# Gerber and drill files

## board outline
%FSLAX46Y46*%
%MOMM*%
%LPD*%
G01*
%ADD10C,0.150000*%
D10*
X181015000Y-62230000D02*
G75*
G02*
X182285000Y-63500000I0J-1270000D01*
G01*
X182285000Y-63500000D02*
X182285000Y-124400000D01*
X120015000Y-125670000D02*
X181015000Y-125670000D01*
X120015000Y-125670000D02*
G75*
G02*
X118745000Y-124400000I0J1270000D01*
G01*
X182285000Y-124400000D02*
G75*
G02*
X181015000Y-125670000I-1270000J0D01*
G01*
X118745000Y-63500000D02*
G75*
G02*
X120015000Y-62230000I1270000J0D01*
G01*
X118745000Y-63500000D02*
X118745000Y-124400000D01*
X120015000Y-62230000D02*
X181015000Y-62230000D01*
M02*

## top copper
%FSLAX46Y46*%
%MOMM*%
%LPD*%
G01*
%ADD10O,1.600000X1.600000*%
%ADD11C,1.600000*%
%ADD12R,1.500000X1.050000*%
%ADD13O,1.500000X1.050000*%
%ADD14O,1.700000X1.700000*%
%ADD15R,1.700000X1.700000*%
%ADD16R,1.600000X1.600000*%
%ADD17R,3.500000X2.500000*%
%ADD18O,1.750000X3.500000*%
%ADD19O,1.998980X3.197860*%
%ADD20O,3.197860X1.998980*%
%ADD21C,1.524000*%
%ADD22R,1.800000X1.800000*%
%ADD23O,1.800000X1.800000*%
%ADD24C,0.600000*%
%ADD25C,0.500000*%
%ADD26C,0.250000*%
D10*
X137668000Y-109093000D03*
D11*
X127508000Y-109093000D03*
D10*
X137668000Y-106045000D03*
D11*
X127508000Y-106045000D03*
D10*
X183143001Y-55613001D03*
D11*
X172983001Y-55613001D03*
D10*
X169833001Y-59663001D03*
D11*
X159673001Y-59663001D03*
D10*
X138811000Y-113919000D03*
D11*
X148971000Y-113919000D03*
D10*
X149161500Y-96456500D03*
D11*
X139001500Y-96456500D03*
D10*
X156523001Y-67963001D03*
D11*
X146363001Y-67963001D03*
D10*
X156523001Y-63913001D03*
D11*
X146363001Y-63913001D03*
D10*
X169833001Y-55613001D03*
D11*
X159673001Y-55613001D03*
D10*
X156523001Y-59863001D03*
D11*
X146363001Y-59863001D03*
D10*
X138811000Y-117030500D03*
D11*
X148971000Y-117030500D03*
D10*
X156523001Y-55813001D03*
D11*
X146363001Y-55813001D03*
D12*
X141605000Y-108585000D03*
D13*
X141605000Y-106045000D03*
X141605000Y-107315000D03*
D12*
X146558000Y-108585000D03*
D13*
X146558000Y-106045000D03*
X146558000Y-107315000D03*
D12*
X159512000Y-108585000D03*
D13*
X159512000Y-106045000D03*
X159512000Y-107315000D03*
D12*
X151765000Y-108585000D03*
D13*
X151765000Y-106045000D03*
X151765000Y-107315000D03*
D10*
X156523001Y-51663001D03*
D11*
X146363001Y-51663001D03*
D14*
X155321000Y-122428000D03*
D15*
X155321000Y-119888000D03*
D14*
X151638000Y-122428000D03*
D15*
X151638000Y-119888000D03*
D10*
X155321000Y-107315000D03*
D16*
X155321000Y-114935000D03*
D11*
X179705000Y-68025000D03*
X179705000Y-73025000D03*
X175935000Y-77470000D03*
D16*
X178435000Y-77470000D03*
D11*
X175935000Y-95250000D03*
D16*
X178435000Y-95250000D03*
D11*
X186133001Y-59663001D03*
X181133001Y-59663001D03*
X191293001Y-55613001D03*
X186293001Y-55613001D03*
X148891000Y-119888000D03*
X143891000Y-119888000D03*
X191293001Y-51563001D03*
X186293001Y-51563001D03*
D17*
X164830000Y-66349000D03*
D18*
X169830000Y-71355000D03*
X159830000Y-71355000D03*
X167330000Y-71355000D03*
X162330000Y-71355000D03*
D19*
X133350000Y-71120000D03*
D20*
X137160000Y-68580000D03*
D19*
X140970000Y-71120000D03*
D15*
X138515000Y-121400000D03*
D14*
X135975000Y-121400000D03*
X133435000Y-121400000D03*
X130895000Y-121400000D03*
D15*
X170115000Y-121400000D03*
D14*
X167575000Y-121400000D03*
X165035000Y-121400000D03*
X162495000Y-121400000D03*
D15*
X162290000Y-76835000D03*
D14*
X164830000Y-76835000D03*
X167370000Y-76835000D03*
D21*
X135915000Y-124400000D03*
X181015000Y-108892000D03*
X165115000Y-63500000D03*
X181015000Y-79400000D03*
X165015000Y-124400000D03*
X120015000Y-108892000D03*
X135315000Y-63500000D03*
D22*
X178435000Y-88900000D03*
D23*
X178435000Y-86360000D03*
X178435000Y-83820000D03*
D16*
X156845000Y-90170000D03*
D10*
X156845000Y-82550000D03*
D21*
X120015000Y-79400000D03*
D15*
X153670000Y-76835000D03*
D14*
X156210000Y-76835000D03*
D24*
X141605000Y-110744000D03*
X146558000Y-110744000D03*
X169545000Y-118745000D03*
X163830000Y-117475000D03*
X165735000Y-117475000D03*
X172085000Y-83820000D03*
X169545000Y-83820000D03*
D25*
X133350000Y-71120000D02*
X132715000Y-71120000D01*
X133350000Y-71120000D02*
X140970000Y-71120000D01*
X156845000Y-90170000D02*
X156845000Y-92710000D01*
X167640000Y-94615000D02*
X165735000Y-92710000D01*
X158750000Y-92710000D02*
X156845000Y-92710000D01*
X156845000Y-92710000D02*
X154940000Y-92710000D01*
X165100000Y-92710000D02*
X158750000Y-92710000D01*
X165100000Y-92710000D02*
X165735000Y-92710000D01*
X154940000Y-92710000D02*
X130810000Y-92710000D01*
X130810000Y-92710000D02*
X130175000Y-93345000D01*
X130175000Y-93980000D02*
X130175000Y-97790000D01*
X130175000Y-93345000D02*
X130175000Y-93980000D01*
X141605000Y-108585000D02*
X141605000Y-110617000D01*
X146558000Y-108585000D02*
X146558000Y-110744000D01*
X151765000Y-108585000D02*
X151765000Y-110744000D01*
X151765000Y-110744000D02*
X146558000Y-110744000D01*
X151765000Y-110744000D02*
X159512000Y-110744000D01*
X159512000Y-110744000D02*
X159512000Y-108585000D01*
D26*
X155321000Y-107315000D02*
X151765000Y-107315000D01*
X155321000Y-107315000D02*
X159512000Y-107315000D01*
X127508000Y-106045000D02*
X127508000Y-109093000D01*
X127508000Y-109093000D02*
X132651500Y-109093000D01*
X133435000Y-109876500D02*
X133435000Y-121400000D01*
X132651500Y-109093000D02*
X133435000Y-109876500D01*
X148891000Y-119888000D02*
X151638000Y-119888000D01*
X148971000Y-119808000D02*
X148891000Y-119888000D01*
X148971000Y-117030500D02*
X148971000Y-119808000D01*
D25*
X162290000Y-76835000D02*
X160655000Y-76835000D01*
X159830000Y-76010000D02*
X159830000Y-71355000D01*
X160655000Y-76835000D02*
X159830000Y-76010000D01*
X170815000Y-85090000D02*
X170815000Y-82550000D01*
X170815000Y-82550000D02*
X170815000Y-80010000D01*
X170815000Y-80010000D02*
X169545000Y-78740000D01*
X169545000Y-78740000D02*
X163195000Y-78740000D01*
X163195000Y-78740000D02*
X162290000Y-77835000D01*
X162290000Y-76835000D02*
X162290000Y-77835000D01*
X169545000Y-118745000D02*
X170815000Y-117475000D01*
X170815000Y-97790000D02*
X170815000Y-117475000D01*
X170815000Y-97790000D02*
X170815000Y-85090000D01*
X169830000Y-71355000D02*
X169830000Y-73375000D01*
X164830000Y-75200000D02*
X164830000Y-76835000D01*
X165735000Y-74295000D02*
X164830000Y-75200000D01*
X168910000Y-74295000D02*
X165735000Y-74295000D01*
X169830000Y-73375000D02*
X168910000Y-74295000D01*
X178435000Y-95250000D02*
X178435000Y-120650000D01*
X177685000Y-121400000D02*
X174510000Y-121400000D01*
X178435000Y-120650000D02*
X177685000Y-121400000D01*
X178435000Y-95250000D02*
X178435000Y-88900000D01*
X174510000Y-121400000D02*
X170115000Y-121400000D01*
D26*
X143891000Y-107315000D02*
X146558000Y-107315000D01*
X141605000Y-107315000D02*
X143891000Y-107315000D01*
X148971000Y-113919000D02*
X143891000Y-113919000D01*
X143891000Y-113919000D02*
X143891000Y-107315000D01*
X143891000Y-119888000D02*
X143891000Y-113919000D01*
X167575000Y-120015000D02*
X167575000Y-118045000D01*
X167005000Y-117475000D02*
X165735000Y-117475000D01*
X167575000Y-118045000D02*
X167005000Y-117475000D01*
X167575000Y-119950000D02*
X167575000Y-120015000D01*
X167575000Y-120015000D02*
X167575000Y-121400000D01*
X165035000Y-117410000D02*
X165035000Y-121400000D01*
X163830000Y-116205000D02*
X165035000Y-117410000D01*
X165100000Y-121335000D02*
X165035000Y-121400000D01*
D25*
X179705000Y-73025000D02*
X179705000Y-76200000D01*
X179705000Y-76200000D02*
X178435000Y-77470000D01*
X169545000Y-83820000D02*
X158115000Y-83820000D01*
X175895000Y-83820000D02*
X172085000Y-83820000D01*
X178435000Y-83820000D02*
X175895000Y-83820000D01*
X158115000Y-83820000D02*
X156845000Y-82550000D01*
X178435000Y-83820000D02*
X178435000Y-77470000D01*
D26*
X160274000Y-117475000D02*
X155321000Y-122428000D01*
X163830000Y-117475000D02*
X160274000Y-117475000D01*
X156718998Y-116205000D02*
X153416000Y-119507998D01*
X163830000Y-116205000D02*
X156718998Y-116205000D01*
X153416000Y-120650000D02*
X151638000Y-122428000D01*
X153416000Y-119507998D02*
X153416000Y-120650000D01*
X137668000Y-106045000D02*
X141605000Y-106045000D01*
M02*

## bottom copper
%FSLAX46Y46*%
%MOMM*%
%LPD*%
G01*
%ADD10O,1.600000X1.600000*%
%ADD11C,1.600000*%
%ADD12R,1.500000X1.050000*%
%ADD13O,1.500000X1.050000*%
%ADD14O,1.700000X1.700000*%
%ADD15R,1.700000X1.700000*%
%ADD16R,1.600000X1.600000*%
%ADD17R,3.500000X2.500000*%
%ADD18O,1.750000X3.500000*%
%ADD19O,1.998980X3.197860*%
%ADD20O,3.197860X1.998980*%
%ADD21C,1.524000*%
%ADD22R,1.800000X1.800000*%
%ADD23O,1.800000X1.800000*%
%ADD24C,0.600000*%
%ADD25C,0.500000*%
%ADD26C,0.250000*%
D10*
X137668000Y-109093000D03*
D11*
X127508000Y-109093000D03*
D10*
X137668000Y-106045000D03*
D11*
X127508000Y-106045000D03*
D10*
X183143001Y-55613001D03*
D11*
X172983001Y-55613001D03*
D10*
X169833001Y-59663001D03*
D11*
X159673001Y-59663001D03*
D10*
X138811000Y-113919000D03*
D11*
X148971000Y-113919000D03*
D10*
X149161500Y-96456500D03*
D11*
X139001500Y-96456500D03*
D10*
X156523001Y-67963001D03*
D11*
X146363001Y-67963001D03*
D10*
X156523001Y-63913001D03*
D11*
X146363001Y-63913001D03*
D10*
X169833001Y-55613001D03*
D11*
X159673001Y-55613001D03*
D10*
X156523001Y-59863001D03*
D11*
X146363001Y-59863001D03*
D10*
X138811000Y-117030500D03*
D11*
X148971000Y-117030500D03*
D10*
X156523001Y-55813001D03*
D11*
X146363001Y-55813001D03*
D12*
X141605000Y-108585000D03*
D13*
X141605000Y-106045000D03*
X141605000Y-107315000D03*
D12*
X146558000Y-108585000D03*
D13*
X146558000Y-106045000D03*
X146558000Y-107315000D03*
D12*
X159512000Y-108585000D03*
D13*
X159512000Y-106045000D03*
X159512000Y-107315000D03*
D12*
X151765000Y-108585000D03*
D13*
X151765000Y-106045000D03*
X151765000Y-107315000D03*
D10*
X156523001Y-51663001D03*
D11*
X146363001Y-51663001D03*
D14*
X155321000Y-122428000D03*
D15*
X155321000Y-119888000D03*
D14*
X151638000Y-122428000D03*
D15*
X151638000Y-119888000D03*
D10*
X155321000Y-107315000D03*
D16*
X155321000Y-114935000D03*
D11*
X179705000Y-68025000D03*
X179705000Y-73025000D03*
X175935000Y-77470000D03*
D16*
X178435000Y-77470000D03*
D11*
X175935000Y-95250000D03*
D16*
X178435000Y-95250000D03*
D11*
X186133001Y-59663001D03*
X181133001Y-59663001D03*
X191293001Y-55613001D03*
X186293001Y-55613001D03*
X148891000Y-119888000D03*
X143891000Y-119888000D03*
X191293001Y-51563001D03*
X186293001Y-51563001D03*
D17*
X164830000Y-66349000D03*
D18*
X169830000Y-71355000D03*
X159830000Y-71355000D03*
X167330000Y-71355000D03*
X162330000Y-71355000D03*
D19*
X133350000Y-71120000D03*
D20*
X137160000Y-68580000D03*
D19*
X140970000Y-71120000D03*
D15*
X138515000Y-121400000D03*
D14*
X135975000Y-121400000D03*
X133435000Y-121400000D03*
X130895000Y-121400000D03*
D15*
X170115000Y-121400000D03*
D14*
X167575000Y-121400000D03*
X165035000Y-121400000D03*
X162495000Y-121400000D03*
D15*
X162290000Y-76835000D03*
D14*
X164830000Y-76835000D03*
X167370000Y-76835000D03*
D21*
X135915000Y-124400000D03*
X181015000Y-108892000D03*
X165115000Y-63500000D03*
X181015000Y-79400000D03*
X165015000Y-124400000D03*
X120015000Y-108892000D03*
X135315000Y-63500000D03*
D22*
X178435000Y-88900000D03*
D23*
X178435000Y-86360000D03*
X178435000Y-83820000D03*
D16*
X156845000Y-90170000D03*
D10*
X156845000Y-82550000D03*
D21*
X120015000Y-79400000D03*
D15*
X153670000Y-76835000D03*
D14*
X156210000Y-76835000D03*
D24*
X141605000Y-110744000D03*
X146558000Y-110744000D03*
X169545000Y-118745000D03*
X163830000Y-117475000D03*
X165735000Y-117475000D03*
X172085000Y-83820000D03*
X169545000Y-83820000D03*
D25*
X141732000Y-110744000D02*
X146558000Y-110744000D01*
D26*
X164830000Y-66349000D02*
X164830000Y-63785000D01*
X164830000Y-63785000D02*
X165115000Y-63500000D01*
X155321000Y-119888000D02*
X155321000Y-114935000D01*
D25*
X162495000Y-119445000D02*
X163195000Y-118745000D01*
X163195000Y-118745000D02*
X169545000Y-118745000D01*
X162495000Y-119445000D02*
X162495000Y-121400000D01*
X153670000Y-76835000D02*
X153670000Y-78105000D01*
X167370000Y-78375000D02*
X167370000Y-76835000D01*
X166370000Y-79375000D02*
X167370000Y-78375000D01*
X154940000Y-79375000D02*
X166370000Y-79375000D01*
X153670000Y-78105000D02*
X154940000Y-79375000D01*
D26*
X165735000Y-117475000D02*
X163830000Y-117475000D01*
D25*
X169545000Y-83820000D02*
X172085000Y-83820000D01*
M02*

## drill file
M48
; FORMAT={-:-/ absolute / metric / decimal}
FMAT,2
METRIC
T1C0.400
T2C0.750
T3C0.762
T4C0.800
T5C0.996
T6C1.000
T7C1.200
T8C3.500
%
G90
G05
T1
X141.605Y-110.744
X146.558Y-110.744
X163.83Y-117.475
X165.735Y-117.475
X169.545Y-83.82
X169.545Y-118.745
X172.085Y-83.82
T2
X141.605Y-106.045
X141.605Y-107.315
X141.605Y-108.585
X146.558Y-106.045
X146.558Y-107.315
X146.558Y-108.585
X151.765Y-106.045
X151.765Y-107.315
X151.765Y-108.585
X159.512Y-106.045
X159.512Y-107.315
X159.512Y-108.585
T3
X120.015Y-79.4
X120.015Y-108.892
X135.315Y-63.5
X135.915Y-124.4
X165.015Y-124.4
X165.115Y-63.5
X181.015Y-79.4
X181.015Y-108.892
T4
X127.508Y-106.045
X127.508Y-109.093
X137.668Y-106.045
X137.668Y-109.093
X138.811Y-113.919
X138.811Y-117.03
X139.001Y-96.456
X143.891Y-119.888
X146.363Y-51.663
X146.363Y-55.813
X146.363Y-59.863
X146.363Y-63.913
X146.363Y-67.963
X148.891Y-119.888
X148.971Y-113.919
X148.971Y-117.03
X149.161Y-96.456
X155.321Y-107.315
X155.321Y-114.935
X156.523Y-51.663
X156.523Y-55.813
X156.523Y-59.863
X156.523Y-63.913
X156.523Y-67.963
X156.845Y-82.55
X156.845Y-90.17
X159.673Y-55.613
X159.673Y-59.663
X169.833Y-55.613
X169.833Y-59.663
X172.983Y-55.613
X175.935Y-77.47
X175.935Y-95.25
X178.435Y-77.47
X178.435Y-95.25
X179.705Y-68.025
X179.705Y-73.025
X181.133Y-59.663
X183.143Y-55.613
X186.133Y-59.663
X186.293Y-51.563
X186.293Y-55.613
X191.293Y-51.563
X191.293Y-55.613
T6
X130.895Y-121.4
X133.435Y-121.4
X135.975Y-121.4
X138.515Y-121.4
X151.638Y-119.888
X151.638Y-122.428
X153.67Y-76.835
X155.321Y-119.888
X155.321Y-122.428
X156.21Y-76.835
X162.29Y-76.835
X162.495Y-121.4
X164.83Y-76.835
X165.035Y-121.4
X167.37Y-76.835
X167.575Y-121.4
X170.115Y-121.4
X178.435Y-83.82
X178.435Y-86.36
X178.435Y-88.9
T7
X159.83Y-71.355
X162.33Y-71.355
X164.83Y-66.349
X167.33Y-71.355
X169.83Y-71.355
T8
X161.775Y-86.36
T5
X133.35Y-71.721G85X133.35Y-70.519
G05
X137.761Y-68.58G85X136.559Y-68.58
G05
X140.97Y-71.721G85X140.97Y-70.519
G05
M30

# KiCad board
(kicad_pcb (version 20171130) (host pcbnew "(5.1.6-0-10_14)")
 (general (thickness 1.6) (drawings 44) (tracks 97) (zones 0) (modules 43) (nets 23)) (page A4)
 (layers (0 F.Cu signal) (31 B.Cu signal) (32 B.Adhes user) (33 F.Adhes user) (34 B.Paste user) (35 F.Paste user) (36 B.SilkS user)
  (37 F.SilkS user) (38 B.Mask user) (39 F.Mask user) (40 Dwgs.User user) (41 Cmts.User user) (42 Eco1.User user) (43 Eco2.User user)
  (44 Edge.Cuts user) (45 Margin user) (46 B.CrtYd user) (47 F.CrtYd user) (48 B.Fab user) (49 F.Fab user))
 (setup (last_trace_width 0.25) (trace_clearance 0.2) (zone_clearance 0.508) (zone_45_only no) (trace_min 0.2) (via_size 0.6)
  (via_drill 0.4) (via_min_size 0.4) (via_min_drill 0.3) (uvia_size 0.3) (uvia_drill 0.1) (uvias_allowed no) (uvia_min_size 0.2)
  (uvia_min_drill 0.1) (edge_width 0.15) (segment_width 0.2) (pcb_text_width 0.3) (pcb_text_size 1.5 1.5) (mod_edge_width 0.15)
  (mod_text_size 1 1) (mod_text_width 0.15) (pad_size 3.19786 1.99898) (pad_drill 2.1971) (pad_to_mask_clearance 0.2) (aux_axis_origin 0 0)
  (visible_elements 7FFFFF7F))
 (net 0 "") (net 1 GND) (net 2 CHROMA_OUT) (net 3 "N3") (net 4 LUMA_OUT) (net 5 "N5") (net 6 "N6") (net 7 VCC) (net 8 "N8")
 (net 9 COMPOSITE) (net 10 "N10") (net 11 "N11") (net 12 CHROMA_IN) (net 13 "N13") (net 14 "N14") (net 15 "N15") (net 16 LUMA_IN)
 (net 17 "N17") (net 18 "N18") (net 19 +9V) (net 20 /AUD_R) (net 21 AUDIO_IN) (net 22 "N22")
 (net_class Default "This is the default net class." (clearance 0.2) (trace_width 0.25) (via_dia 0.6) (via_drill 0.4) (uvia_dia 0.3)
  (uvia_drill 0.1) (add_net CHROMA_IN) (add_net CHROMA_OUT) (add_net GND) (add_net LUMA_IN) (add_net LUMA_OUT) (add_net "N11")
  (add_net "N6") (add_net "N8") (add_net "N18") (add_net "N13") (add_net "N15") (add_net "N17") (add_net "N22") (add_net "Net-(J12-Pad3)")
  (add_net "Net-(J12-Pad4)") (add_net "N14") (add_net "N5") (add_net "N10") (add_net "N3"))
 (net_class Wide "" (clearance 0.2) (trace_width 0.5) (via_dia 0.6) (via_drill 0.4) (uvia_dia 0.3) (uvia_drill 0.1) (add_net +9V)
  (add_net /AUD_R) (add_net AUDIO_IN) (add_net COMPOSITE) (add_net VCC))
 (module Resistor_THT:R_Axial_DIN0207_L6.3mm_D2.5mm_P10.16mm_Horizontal (layer F.Cu) (at 127.508 109.093)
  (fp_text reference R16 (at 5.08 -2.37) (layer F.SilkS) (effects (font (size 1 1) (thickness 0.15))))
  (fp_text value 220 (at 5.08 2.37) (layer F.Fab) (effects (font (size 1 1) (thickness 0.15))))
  (pad 2 thru_hole oval (at 10.16 0) (size 1.6 1.6) (drill 0.8) (layers *.Cu *.Mask) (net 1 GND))
  (pad 1 thru_hole circle (at 0 0) (size 1.6 1.6) (drill 0.8) (layers *.Cu *.Mask) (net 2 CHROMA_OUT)))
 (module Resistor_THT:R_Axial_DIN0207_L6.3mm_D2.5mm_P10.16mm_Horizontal (layer F.Cu) (at 127.508 106.045)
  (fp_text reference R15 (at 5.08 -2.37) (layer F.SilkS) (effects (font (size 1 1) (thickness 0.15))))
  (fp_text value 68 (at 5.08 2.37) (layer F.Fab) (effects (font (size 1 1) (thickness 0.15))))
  (pad 2 thru_hole oval (at 10.16 0) (size 1.6 1.6) (drill 0.8) (layers *.Cu *.Mask) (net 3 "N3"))
  (pad 1 thru_hole circle (at 0 0) (size 1.6 1.6) (drill 0.8) (layers *.Cu *.Mask) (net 2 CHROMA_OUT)))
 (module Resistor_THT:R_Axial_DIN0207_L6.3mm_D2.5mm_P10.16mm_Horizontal (layer F.Cu) (at 172.983001 55.613001)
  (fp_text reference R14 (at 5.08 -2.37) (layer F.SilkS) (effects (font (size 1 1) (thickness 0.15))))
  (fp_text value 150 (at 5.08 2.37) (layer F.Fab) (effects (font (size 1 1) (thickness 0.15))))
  (pad 2 thru_hole oval (at 10.16 0) (size 1.6 1.6) (drill 0.8) (layers *.Cu *.Mask) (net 1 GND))
  (pad 1 thru_hole circle (at 0 0) (size 1.6 1.6) (drill 0.8) (layers *.Cu *.Mask) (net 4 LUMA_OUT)))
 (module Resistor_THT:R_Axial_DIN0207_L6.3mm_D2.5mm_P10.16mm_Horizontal (layer F.Cu) (at 159.673001 59.663001)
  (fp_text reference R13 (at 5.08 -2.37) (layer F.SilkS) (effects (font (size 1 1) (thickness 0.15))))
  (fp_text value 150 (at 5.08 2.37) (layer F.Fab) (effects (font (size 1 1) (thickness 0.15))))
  (pad 2 thru_hole oval (at 10.16 0) (size 1.6 1.6) (drill 0.8) (layers *.Cu *.Mask) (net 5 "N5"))
  (pad 1 thru_hole circle (at 0 0) (size 1.6 1.6) (drill 0.8) (layers *.Cu *.Mask) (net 4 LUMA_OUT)))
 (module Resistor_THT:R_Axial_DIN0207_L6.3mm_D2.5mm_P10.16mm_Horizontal (layer F.Cu) (at 148.971 113.919 180)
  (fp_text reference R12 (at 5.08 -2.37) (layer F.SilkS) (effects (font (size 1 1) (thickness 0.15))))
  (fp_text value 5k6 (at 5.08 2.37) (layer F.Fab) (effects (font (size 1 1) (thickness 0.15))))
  (pad 2 thru_hole oval (at 10.16 0 180) (size 1.6 1.6) (drill 0.8) (layers *.Cu *.Mask) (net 1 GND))
  (pad 1 thru_hole circle (at 0 0 180) (size 1.6 1.6) (drill 0.8) (layers *.Cu *.Mask) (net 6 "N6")))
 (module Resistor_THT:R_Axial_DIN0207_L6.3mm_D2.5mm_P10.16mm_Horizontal (layer F.Cu) (at 139.0015 96.4565)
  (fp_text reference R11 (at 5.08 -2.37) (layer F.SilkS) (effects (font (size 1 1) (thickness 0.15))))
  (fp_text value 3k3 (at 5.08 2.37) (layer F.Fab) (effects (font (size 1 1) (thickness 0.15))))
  (pad 2 thru_hole oval (at 10.16 0) (size 1.6 1.6) (drill 0.8) (layers *.Cu *.Mask) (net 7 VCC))
  (pad 1 thru_hole circle (at 0 0) (size 1.6 1.6) (drill 0.8) (layers *.Cu *.Mask) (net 6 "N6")))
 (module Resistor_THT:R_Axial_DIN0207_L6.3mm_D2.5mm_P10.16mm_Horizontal (layer F.Cu) (at 146.363001 67.963001)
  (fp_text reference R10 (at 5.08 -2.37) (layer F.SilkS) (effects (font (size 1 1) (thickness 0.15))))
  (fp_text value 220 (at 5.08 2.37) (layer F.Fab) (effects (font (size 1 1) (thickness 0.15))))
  (pad 2 thru_hole oval (at 10.16 0) (size 1.6 1.6) (drill 0.8) (layers *.Cu *.Mask) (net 1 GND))
  (pad 1 thru_hole circle (at 0 0) (size 1.6 1.6) (drill 0.8) (layers *.Cu *.Mask) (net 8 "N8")))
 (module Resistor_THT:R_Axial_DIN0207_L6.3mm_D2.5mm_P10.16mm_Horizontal (layer F.Cu) (at 146.363001 63.913001)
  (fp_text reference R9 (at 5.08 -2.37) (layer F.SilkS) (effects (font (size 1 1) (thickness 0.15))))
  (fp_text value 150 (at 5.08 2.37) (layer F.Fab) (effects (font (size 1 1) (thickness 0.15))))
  (pad 2 thru_hole oval (at 10.16 0) (size 1.6 1.6) (drill 0.8) (layers *.Cu *.Mask) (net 1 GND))
  (pad 1 thru_hole circle (at 0 0) (size 1.6 1.6) (drill 0.8) (layers *.Cu *.Mask) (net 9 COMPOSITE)))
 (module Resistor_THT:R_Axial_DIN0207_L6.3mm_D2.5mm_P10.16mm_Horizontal (layer F.Cu) (at 159.673001 55.613001)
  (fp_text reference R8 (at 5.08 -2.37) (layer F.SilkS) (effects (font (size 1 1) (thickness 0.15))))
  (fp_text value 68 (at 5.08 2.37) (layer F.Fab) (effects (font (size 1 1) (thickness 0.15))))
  (pad 2 thru_hole oval (at 10.16 0) (size 1.6 1.6) (drill 0.8) (layers *.Cu *.Mask) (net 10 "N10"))
  (pad 1 thru_hole circle (at 0 0) (size 1.6 1.6) (drill 0.8) (layers *.Cu *.Mask) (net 8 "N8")))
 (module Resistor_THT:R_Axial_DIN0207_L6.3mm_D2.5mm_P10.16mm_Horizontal (layer F.Cu) (at 146.363001 59.863001)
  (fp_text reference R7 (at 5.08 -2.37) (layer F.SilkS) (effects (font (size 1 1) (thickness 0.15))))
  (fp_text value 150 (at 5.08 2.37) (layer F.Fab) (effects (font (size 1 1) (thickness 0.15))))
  (pad 2 thru_hole oval (at 10.16 0) (size 1.6 1.6) (drill 0.8) (layers *.Cu *.Mask) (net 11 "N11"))
  (pad 1 thru_hole circle (at 0 0) (size 1.6 1.6) (drill 0.8) (layers *.Cu *.Mask) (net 9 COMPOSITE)))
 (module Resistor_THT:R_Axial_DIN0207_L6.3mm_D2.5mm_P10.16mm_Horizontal (layer F.Cu) (at 148.971 117.0305 180)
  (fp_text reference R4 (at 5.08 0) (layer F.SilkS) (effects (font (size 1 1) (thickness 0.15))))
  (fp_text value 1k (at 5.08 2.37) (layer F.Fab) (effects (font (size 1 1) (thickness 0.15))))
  (pad 2 thru_hole oval (at 10.16 0 180) (size 1.6 1.6) (drill 0.8) (layers *.Cu *.Mask) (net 1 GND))
  (pad 1 thru_hole circle (at 0 0 180) (size 1.6 1.6) (drill 0.8) (layers *.Cu *.Mask) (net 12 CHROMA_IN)))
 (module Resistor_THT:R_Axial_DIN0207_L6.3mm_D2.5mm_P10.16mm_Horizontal (layer F.Cu) (at 146.363001 55.813001)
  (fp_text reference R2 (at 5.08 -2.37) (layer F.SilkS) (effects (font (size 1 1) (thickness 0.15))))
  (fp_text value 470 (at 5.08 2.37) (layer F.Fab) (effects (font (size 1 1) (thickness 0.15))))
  (pad 2 thru_hole oval (at 10.16 0) (size 1.6 1.6) (drill 0.8) (layers *.Cu *.Mask) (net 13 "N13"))
  (pad 1 thru_hole circle (at 0 0) (size 1.6 1.6) (drill 0.8) (layers *.Cu *.Mask) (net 7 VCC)))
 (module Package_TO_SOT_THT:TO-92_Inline (layer F.Cu) (at 141.605 108.585 90)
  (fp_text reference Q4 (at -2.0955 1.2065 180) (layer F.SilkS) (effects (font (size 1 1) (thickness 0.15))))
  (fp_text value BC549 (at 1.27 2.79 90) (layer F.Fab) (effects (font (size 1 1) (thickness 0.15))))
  (pad 1 thru_hole rect (at 0 0 90) (size 1.05 1.5) (drill 0.75) (layers *.Cu *.Mask) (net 7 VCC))
  (pad 3 thru_hole oval (at 2.54 0 90) (size 1.05 1.5) (drill 0.75) (layers *.Cu *.Mask) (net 3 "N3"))
  (pad 2 thru_hole oval (at 1.27 0 90) (size 1.05 1.5) (drill 0.75) (layers *.Cu *.Mask) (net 6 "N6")))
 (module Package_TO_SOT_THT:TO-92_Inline (layer F.Cu) (at 146.558 108.585 90)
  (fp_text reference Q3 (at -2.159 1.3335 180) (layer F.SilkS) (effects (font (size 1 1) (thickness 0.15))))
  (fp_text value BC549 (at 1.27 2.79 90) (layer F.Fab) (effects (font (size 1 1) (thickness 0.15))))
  (pad 1 thru_hole rect (at 0 0 90) (size 1.05 1.5) (drill 0.75) (layers *.Cu *.Mask) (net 7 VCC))
  (pad 3 thru_hole oval (at 2.54 0 90) (size 1.05 1.5) (drill 0.75) (layers *.Cu *.Mask) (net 10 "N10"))
  (pad 2 thru_hole oval (at 1.27 0 90) (size 1.05 1.5) (drill 0.75) (layers *.Cu *.Mask) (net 6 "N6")))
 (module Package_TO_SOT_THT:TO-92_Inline (layer F.Cu) (at 159.512 108.585 90)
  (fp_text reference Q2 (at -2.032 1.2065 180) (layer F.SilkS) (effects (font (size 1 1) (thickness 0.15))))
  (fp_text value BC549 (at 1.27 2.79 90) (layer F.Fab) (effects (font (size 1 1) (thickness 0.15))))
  (pad 1 thru_hole rect (at 0 0 90) (size 1.05 1.5) (drill 0.75) (layers *.Cu *.Mask) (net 7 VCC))
  (pad 3 thru_hole oval (at 2.54 0 90) (size 1.05 1.5) (drill 0.75) (layers *.Cu *.Mask) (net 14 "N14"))
  (pad 2 thru_hole oval (at 1.27 0 90) (size 1.05 1.5) (drill 0.75) (layers *.Cu *.Mask) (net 13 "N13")))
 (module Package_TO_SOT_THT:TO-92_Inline (layer F.Cu) (at 151.765 108.585 90)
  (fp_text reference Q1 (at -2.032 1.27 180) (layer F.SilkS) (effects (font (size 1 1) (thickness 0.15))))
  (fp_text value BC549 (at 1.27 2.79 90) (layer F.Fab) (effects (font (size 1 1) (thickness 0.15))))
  (pad 1 thru_hole rect (at 0 0 90) (size 1.05 1.5) (drill 0.75) (layers *.Cu *.Mask) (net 7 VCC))
  (pad 3 thru_hole oval (at 2.54 0 90) (size 1.05 1.5) (drill 0.75) (layers *.Cu *.Mask) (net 5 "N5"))
  (pad 2 thru_hole oval (at 1.27 0 90) (size 1.05 1.5) (drill 0.75) (layers *.Cu *.Mask) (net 13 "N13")))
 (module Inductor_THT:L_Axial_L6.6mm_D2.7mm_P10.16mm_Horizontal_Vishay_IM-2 (layer F.Cu) (at 146.363001 51.663001)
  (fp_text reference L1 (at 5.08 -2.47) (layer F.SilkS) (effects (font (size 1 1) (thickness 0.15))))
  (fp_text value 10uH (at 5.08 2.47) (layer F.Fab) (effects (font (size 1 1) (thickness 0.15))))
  (pad 2 thru_hole oval (at 10.16 0) (size 1.6 1.6) (drill 0.8) (layers *.Cu *.Mask) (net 14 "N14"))
  (pad 1 thru_hole circle (at 0 0) (size 1.6 1.6) (drill 0.8) (layers *.Cu *.Mask) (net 11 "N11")))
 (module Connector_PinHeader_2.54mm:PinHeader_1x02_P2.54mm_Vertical (layer F.Cu) (at 155.321 119.888)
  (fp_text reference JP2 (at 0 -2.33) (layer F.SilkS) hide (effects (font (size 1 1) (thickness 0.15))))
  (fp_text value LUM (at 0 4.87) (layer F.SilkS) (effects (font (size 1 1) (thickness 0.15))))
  (pad 2 thru_hole oval (at 0 2.54) (size 1.7 1.7) (drill 1) (layers *.Cu *.Mask) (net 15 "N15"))
  (pad 1 thru_hole rect (at 0 0) (size 1.7 1.7) (drill 1) (layers *.Cu *.Mask) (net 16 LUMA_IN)))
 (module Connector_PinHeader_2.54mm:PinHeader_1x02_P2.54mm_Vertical (layer F.Cu) (at 151.638 119.888)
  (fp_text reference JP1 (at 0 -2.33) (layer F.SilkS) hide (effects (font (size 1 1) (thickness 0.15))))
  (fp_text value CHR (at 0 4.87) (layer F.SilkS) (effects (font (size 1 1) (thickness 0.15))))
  (pad 2 thru_hole oval (at 0 2.54) (size 1.7 1.7) (drill 1) (layers *.Cu *.Mask) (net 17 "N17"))
  (pad 1 thru_hole rect (at 0 0) (size 1.7 1.7) (drill 1) (layers *.Cu *.Mask) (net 12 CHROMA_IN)))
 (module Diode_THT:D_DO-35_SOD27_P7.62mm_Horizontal (layer F.Cu) (at 155.321 114.935 90)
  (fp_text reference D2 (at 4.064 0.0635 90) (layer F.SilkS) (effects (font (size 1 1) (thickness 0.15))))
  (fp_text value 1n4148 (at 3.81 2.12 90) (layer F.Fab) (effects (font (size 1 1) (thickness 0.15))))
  (pad 2 thru_hole oval (at 7.62 0 90) (size 1.6 1.6) (drill 0.8) (layers *.Cu *.Mask) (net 13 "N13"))
  (pad 1 thru_hole rect (at 0 0 90) (size 1.6 1.6) (drill 0.8) (layers *.Cu *.Mask) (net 16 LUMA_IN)))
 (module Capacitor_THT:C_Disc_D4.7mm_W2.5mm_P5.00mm (layer F.Cu) (at 179.705 73.025 90)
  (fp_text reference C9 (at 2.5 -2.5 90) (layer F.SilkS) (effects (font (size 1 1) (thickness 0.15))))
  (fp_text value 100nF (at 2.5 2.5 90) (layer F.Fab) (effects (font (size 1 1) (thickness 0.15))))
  (pad 2 thru_hole circle (at 5 0 90) (size 1.6 1.6) (drill 0.8) (layers *.Cu *.Mask) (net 1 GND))
  (pad 1 thru_hole circle (at 0 0 90) (size 1.6 1.6) (drill 0.8) (layers *.Cu *.Mask) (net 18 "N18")))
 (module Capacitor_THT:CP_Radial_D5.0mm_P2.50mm (layer F.Cu) (at 178.435 77.47 180)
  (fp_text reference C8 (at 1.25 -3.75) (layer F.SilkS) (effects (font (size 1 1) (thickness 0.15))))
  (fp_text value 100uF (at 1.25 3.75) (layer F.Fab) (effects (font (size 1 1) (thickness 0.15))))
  (pad 2 thru_hole circle (at 2.5 0 180) (size 1.6 1.6) (drill 0.8) (layers *.Cu *.Mask) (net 1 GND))
  (pad 1 thru_hole rect (at 0 0 180) (size 1.6 1.6) (drill 0.8) (layers *.Cu *.Mask) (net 18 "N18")))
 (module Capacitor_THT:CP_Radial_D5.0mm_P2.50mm (layer F.Cu) (at 178.435 95.25 180)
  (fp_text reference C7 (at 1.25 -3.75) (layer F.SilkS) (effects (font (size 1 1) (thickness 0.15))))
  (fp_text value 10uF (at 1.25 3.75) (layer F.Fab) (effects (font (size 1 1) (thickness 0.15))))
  (pad 2 thru_hole circle (at 2.5 0 180) (size 1.6 1.6) (drill 0.8) (layers *.Cu *.Mask) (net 1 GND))
  (pad 1 thru_hole rect (at 0 0 180) (size 1.6 1.6) (drill 0.8) (layers *.Cu *.Mask) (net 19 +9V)))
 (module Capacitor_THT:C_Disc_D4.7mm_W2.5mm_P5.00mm (layer F.Cu) (at 181.133001 59.663001)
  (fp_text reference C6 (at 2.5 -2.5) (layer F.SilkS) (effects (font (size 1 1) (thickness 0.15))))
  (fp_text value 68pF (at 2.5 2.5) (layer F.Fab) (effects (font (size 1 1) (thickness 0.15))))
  (pad 2 thru_hole circle (at 5 0) (size 1.6 1.6) (drill 0.8) (layers *.Cu *.Mask) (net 9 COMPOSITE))
  (pad 1 thru_hole circle (at 0 0) (size 1.6 1.6) (drill 0.8) (layers *.Cu *.Mask) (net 8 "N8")))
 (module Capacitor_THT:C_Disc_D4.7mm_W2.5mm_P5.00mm (layer F.Cu) (at 186.293001 55.613001)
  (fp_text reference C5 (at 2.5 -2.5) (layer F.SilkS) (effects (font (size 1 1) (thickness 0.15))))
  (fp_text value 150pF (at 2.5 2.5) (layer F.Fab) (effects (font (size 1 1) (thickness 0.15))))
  (pad 2 thru_hole circle (at 5 0) (size 1.6 1.6) (drill 0.8) (layers *.Cu *.Mask) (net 1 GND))
  (pad 1 thru_hole circle (at 0 0) (size 1.6 1.6) (drill 0.8) (layers *.Cu *.Mask) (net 6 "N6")))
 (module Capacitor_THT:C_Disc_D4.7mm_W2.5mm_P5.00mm (layer F.Cu) (at 143.891 119.888)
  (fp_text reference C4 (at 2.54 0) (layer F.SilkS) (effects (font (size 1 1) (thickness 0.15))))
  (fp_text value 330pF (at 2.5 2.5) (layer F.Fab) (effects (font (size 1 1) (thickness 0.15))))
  (pad 2 thru_hole circle (at 5 0) (size 1.6 1.6) (drill 0.8) (layers *.Cu *.Mask) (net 12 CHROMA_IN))
  (pad 1 thru_hole circle (at 0 0) (size 1.6 1.6) (drill 0.8) (layers *.Cu *.Mask) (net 6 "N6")))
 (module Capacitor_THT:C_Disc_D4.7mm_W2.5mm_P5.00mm (layer F.Cu) (at 186.293001 51.563001)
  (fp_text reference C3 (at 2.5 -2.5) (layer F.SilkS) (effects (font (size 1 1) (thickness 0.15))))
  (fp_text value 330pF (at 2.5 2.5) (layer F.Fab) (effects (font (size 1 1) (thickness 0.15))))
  (pad 2 thru_hole circle (at 5 0) (size 1.6 1.6) (drill 0.8) (layers *.Cu *.Mask) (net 1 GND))
  (pad 1 thru_hole circle (at 0 0) (size 1.6 1.6) (drill 0.8) (layers *.Cu *.Mask) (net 11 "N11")))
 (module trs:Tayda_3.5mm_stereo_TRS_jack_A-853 (layer F.Cu) (at 164.83 67.945)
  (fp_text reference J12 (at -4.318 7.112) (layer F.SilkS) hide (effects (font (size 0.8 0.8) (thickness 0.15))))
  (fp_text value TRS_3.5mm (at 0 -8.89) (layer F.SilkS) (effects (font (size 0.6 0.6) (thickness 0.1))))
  (pad 1 thru_hole rect (at 0 -1.596) (size 3.5 2.5) (drill 1.2) (layers *.Cu *.Mask F.SilkS) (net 1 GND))
  (pad 2 thru_hole oval (at 5 3.41) (size 1.75 3.5) (drill 1.2) (layers *.Cu *.Mask F.SilkS) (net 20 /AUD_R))
  (pad 5 thru_hole oval (at -5 3.41) (size 1.75 3.5) (drill 1.2) (layers *.Cu *.Mask F.SilkS) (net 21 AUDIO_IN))
  (pad 3 thru_hole oval (at 2.5 3.41) (size 1.75 3.5) (drill 1.2) (layers *.Cu *.Mask F.SilkS))
  (pad 4 thru_hole oval (at -2.5 3.41) (size 1.75 3.5) (drill 1.2) (layers *.Cu *.Mask F.SilkS)))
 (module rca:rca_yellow (layer F.Cu) (at 137.16 67.31 180)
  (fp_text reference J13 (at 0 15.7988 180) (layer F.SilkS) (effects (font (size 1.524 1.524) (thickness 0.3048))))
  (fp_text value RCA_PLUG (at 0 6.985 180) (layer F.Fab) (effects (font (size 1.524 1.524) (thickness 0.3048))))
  (pad 2 thru_hole oval (at 3.81 -3.81 180) (size 1.99898 3.19786) (drill oval 0.99568 2.1971) (layers *.Cu *.Mask F.SilkS)
   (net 9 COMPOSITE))
  (pad 1 thru_hole oval (at 0 -1.27 180) (size 3.19786 1.99898) (drill oval 2.1971 0.99568) (layers *.Cu *.Mask F.SilkS) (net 1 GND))
  (pad 2 thru_hole oval (at -3.81 -3.81 180) (size 1.99898 3.19786) (drill oval 0.99568 2.1971) (layers *.Cu *.Mask F.SilkS)
   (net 9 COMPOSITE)))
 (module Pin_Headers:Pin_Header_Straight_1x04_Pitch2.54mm (layer F.Cu) (at 138.515 121.4 270)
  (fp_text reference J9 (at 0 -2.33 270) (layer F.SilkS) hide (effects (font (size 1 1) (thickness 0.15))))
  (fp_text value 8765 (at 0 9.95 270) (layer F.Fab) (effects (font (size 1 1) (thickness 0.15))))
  (pad 1 thru_hole rect (at 0 0 270) (size 1.7 1.7) (drill 1) (layers *.Cu *.Mask) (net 9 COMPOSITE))
  (pad 2 thru_hole oval (at 0 2.54 270) (size 1.7 1.7) (drill 1) (layers *.Cu *.Mask) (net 4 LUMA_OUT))
  (pad 3 thru_hole oval (at 0 5.08 270) (size 1.7 1.7) (drill 1) (layers *.Cu *.Mask) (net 2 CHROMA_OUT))
  (pad 4 thru_hole oval (at 0 7.62 270) (size 1.7 1.7) (drill 1) (layers *.Cu *.Mask) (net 1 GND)))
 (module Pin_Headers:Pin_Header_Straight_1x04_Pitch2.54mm (layer F.Cu) (at 170.115 121.4 270)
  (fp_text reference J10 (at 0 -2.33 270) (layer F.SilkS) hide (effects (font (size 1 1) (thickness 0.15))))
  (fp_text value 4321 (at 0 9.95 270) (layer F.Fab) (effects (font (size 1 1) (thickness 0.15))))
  (pad 1 thru_hole rect (at 0 0 270) (size 1.7 1.7) (drill 1) (layers *.Cu *.Mask) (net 19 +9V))
  (pad 2 thru_hole oval (at 0 2.54 270) (size 1.7 1.7) (drill 1) (layers *.Cu *.Mask) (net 15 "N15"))
  (pad 3 thru_hole oval (at 0 5.08 270) (size 1.7 1.7) (drill 1) (layers *.Cu *.Mask) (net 17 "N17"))
  (pad 4 thru_hole oval (at 0 7.62 270) (size 1.7 1.7) (drill 1) (layers *.Cu *.Mask) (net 21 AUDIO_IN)))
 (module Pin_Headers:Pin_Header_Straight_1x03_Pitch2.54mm (layer F.Cu) (at 162.29 76.835 90)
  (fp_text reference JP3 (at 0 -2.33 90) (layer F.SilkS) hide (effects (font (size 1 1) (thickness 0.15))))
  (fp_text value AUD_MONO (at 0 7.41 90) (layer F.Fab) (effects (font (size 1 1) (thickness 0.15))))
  (pad 1 thru_hole rect (at 0 0 90) (size 1.7 1.7) (drill 1) (layers *.Cu *.Mask) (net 21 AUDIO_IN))
  (pad 2 thru_hole oval (at 0 2.54 90) (size 1.7 1.7) (drill 1) (layers *.Cu *.Mask) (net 20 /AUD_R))
  (pad 3 thru_hole oval (at 0 5.08 90) (size 1.7 1.7) (drill 1) (layers *.Cu *.Mask) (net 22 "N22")))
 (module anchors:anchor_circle (layer F.Cu) (at 135.89 124.46)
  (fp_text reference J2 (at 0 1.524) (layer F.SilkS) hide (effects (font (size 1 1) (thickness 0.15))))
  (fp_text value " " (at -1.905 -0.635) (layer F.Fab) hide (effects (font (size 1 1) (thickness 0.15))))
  (pad 1 thru_hole circle (at 0.025 -0.06) (size 1.524 1.524) (drill 0.762) (layers *.Cu *.Mask) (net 1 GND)))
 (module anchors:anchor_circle (layer F.Cu) (at 180.975 109.4)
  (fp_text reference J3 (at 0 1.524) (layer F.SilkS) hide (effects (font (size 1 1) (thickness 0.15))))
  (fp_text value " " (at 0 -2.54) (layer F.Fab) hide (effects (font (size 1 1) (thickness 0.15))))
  (pad 1 thru_hole circle (at 0.04 -0.508) (size 1.524 1.524) (drill 0.762) (layers *.Cu *.Mask) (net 1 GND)))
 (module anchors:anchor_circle (layer F.Cu) (at 168.91 63.5)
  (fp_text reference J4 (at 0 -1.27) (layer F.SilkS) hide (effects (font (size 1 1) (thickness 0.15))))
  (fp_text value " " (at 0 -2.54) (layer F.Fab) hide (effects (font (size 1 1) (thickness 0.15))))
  (pad 1 thru_hole circle (at -3.795 0) (size 1.524 1.524) (drill 0.762) (layers *.Cu *.Mask) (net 1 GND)))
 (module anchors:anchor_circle (layer F.Cu) (at 180.975 79.375)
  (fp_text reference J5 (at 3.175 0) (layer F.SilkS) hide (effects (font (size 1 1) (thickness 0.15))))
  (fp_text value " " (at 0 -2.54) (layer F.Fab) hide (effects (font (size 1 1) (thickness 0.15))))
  (pad 1 thru_hole circle (at 0.04 0.025) (size 1.524 1.524) (drill 0.762) (layers *.Cu *.Mask) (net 1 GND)))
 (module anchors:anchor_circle (layer F.Cu) (at 165.015 126.365)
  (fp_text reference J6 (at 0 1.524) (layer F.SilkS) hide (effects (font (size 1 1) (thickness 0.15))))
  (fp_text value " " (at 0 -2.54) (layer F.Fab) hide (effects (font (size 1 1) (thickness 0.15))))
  (pad 1 thru_hole circle (at 0 -1.965) (size 1.524 1.524) (drill 0.762) (layers *.Cu *.Mask) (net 1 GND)))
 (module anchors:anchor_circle (layer F.Cu) (at 120.015 113.665)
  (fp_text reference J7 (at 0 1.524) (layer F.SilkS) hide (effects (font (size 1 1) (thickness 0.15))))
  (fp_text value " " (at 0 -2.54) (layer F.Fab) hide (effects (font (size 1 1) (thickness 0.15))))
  (pad 1 thru_hole circle (at 0 -4.773) (size 1.524 1.524) (drill 0.762) (layers *.Cu *.Mask) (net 1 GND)))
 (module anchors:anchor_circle (layer F.Cu) (at 135.315 63.5)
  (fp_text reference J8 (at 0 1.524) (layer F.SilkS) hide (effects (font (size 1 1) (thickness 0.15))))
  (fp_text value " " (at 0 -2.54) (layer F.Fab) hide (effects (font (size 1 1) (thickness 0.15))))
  (pad 1 thru_hole circle (at 0 0) (size 1.524 1.524) (drill 0.762) (layers *.Cu *.Mask) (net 1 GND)))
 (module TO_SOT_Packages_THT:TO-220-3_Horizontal (layer F.Cu) (at 178.435 88.9 90)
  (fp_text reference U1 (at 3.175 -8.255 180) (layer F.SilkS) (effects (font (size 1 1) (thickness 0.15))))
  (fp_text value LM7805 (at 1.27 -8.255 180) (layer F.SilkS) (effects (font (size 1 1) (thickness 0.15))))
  (pad 0 np_thru_hole oval (at 2.54 -16.66 90) (size 3.5 3.5) (drill 3.5) (layers *.Cu *.Mask))
  (pad 1 thru_hole rect (at 0 0 90) (size 1.8 1.8) (drill 1) (layers *.Cu *.Mask) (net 19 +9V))
  (pad 2 thru_hole oval (at 2.54 0 90) (size 1.8 1.8) (drill 1) (layers *.Cu *.Mask) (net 1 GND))
  (pad 3 thru_hole oval (at 5.08 0 90) (size 1.8 1.8) (drill 1) (layers *.Cu *.Mask) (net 18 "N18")))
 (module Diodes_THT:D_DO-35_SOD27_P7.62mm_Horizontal (layer F.Cu) (at 156.845 90.17 90)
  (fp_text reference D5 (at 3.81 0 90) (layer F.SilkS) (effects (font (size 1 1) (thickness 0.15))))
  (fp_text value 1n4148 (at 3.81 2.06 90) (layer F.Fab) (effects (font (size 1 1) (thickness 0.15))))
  (pad 1 thru_hole rect (at 0 0 90) (size 1.6 1.6) (drill 0.8) (layers *.Cu *.Mask) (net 7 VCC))
  (pad 2 thru_hole oval (at 7.62 0 90) (size 1.6 1.6) (drill 0.8) (layers *.Cu *.Mask) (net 18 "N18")))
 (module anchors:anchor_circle (layer F.Cu) (at 120.015 79.375)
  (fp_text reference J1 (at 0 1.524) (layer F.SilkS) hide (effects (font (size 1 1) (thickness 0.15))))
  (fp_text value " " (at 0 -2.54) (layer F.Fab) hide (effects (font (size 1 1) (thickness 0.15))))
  (pad 1 thru_hole circle (at 0 0.025) (size 1.524 1.524) (drill 0.762) (layers *.Cu *.Mask) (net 1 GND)))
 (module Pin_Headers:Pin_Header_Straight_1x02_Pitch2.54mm (layer F.Cu) (at 153.67 76.835 90)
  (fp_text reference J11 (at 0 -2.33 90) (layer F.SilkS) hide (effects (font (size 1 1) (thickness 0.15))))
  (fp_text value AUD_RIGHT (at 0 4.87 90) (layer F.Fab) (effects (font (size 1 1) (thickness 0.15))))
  (pad 1 thru_hole rect (at 0 0 90) (size 1.7 1.7) (drill 1) (layers *.Cu *.Mask) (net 22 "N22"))
  (pad 2 thru_hole oval (at 0 2.54 90) (size 1.7 1.7) (drill 1) (layers *.Cu *.Mask) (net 1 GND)))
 (gr_arc (start 181.015 63.5) (end 181.015 62.23) (angle 90) (layer Edge.Cuts) (width 0.15))
 (gr_line (start 182.285 63.5) (end 182.285 124.4) (angle 90) (layer Edge.Cuts) (width 0.15))
 (gr_line (start 120.015 125.67) (end 181.015 125.67) (angle 90) (layer Edge.Cuts) (width 0.15))
 (gr_arc (start 120.015 124.4) (end 120.015 125.67) (angle 90) (layer Edge.Cuts) (width 0.15))
 (gr_arc (start 181.015 124.4) (end 182.285 124.4) (angle 90) (layer Edge.Cuts) (width 0.15))
 (gr_arc (start 120.015 63.5) (end 118.745 63.5) (angle 90) (layer Edge.Cuts) (width 0.15))
 (gr_line (start 118.745 63.5) (end 118.745 124.4) (angle 90) (layer Edge.Cuts) (width 0.15))
 (gr_line (start 120.015 62.23) (end 181.015 62.23) (angle 90) (layer Edge.Cuts) (width 0.15))
 (via (at 141.605 110.744) (size 0.6) (drill 0.4) (layers F.Cu B.Cu) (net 7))
 (via (at 146.558 110.744) (size 0.6) (drill 0.4) (layers F.Cu B.Cu) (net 7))
 (segment (start 141.732 110.744) (end 146.558 110.744) (width 0.5) (layer B.Cu) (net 7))
 (segment (start 164.83 66.349) (end 164.83 63.785) (width 0.25) (layer B.Cu) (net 1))
 (segment (start 164.83 63.785) (end 165.115 63.5) (width 0.25) (layer B.Cu) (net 1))
 (segment (start 133.35 71.12) (end 132.715 71.12) (width 0.5) (layer F.Cu) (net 9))
 (segment (start 133.35 71.12) (end 140.97 71.12) (width 0.5) (layer F.Cu) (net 9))
 (segment (start 156.845 90.17) (end 156.845 92.71) (width 0.5) (layer F.Cu) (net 7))
 (segment (start 167.64 94.615) (end 165.735 92.71) (width 0.5) (layer F.Cu) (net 7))
 (segment (start 158.75 92.71) (end 156.845 92.71) (width 0.5) (layer F.Cu) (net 7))
 (segment (start 156.845 92.71) (end 154.94 92.71) (width 0.5) (layer F.Cu) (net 7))
 (segment (start 165.1 92.71) (end 158.75 92.71) (width 0.5) (layer F.Cu) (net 7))
 (segment (start 165.1 92.71) (end 165.735 92.71) (width 0.5) (layer F.Cu) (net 7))
 (segment (start 154.94 92.71) (end 130.81 92.71) (width 0.5) (layer F.Cu) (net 7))
 (segment (start 130.81 92.71) (end 130.175 93.345) (width 0.5) (layer F.Cu) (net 7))
 (segment (start 130.175 93.98) (end 130.175 97.79) (width 0.5) (layer F.Cu) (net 7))
 (segment (start 130.175 93.345) (end 130.175 93.98) (width 0.5) (layer F.Cu) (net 7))
 (segment (start 141.605 108.585) (end 141.605 110.617) (width 0.5) (layer F.Cu) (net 7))
 (segment (start 146.558 108.585) (end 146.558 110.744) (width 0.5) (layer F.Cu) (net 7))
 (segment (start 151.765 108.585) (end 151.765 110.744) (width 0.5) (layer F.Cu) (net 7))
 (segment (start 151.765 110.744) (end 146.558 110.744) (width 0.5) (layer F.Cu) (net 7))
 (segment (start 151.765 110.744) (end 159.512 110.744) (width 0.5) (layer F.Cu) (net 7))
 (segment (start 159.512 110.744) (end 159.512 108.585) (width 0.5) (layer F.Cu) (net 7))
 (segment (start 155.321 119.888) (end 155.321 114.935) (width 0.25) (layer B.Cu) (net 16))
 (segment (start 155.321 107.315) (end 151.765 107.315) (width 0.25) (layer F.Cu) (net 13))
 (segment (start 155.321 107.315) (end 159.512 107.315) (width 0.25) (layer F.Cu) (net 13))
 (segment (start 127.508 106.045) (end 127.508 109.093) (width 0.25) (layer F.Cu) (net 2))
 (segment (start 127.508 109.093) (end 132.6515 109.093) (width 0.25) (layer F.Cu) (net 2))
 (segment (start 133.435 109.8765) (end 133.435 121.4) (width 0.25) (layer F.Cu) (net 2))
 (segment (start 132.6515 109.093) (end 133.435 109.8765) (width 0.25) (layer F.Cu) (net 2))
 (segment (start 148.891 119.888) (end 151.638 119.888) (width 0.25) (layer F.Cu) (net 12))
 (segment (start 148.971 119.808) (end 148.891 119.888) (width 0.25) (layer F.Cu) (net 12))
 (segment (start 148.971 117.0305) (end 148.971 119.808) (width 0.25) (layer F.Cu) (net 12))
 (segment (start 162.29 76.835) (end 160.655 76.835) (width 0.5) (layer F.Cu) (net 21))
 (segment (start 159.83 76.01) (end 159.83 71.355) (width 0.5) (layer F.Cu) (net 21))
 (segment (start 160.655 76.835) (end 159.83 76.01) (width 0.5) (layer F.Cu) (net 21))
 (segment (start 170.815 85.09) (end 170.815 82.55) (width 0.5) (layer F.Cu) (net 21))
 (segment (start 170.815 82.55) (end 170.815 80.01) (width 0.5) (layer F.Cu) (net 21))
 (segment (start 170.815 80.01) (end 169.545 78.74) (width 0.5) (layer F.Cu) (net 21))
 (segment (start 169.545 78.74) (end 163.195 78.74) (width 0.5) (layer F.Cu) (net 21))
 (segment (start 163.195 78.74) (end 162.29 77.835) (width 0.5) (layer F.Cu) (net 21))
 (segment (start 162.29 76.835) (end 162.29 77.835) (width 0.5) (layer F.Cu) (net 21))
 (segment (start 169.545 118.745) (end 170.815 117.475) (width 0.5) (layer F.Cu) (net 21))
 (segment (start 162.495 119.445) (end 163.195 118.745) (width 0.5) (layer B.Cu) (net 21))
 (segment (start 163.195 118.745) (end 169.545 118.745) (width 0.5) (layer B.Cu) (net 21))
 (via (at 169.545 118.745) (size 0.6) (drill 0.4) (layers F.Cu B.Cu) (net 21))
 (segment (start 170.815 97.79) (end 170.815 117.475) (width 0.5) (layer F.Cu) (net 21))
 (segment (start 162.495 119.445) (end 162.495 121.4) (width 0.5) (layer B.Cu) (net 21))
 (segment (start 170.815 97.79) (end 170.815 85.09) (width 0.5) (layer F.Cu) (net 21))
 (segment (start 153.67 76.835) (end 153.67 78.105) (width 0.5) (layer B.Cu) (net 22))
 (segment (start 167.37 78.375) (end 167.37 76.835) (width 0.5) (layer B.Cu) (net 22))
 (segment (start 166.37 79.375) (end 167.37 78.375) (width 0.5) (layer B.Cu) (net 22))
 (segment (start 154.94 79.375) (end 166.37 79.375) (width 0.5) (layer B.Cu) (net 22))
 (segment (start 153.67 78.105) (end 154.94 79.375) (width 0.5) (layer B.Cu) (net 22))
 (segment (start 169.83 71.355) (end 169.83 73.375) (width 0.5) (layer F.Cu) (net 20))
 (segment (start 164.83 75.2) (end 164.83 76.835) (width 0.5) (layer F.Cu) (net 20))
 (segment (start 165.735 74.295) (end 164.83 75.2) (width 0.5) (layer F.Cu) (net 20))
 (segment (start 168.91 74.295) (end 165.735 74.295) (width 0.5) (layer F.Cu) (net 20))
 (segment (start 169.83 73.375) (end 168.91 74.295) (width 0.5) (layer F.Cu) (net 20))
 (segment (start 178.435 95.25) (end 178.435 120.65) (width 0.5) (layer F.Cu) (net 19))
 (segment (start 177.685 121.4) (end 174.51 121.4) (width 0.5) (layer F.Cu) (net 19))
 (segment (start 178.435 120.65) (end 177.685 121.4) (width 0.5) (layer F.Cu) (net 19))
 (segment (start 178.435 95.25) (end 178.435 88.9) (width 0.5) (layer F.Cu) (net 19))
 (segment (start 174.51 121.4) (end 170.115 121.4) (width 0.5) (layer F.Cu) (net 19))
 (segment (start 143.891 107.315) (end 146.558 107.315) (width 0.25) (layer F.Cu) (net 6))
 (segment (start 141.605 107.315) (end 143.891 107.315) (width 0.25) (layer F.Cu) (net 6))
 (segment (start 148.971 113.919) (end 143.891 113.919) (width 0.25) (layer F.Cu) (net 6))
 (segment (start 143.891 113.919) (end 143.891 107.315) (width 0.25) (layer F.Cu) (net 6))
 (segment (start 143.891 119.888) (end 143.891 113.919) (width 0.25) (layer F.Cu) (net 6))
 (segment (start 167.575 120.015) (end 167.575 118.045) (width 0.25) (layer F.Cu) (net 15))
 (via (at 163.83 117.475) (size 0.6) (drill 0.4) (layers F.Cu B.Cu) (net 15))
 (segment (start 165.735 117.475) (end 163.83 117.475) (width 0.25) (layer B.Cu) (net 15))
 (via (at 165.735 117.475) (size 0.6) (drill 0.4) (layers F.Cu B.Cu) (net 15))
 (segment (start 167.005 117.475) (end 165.735 117.475) (width 0.25) (layer F.Cu) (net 15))
 (segment (start 167.575 118.045) (end 167.005 117.475) (width 0.25) (layer F.Cu) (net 15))
 (segment (start 167.575 119.95) (end 167.575 120.015) (width 0.25) (layer F.Cu) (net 15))
 (segment (start 167.575 120.015) (end 167.575 121.4) (width 0.25) (layer F.Cu) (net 15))
 (segment (start 165.035 117.41) (end 165.035 121.4) (width 0.25) (layer F.Cu) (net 17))
 (segment (start 163.83 116.205) (end 165.035 117.41) (width 0.25) (layer F.Cu) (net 17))
 (segment (start 165.1 121.335) (end 165.035 121.4) (width 0.25) (layer F.Cu) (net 17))
 (segment (start 179.705 73.025) (end 179.705 76.2) (width 0.5) (layer F.Cu) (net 18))
 (segment (start 179.705 76.2) (end 178.435 77.47) (width 0.5) (layer F.Cu) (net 18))
 (segment (start 169.545 83.82) (end 172.085 83.82) (width 0.5) (layer B.Cu) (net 18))
 (segment (start 169.545 83.82) (end 158.115 83.82) (width 0.5) (layer F.Cu) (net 18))
 (segment (start 175.895 83.82) (end 172.085 83.82) (width 0.5) (layer F.Cu) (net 18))
 (segment (start 178.435 83.82) (end 175.895 83.82) (width 0.5) (layer F.Cu) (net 18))
 (segment (start 158.115 83.82) (end 156.845 82.55) (width 0.5) (layer F.Cu) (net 18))
 (via (at 172.085 83.82) (size 0.6) (drill 0.4) (layers F.Cu B.Cu) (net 18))
 (via (at 169.545 83.82) (size 0.6) (drill 0.4) (layers F.Cu B.Cu) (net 18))
 (segment (start 178.435 83.82) (end 178.435 77.47) (width 0.5) (layer F.Cu) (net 18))
 (segment (start 160.274 117.475) (end 155.321 122.428) (width 0.25) (layer F.Cu) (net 15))
 (segment (start 163.83 117.475) (end 160.274 117.475) (width 0.25) (layer F.Cu) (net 15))
 (segment (start 156.718998 116.205) (end 153.416 119.507998) (width 0.25) (layer F.Cu) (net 17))
 (segment (start 163.83 116.205) (end 156.718998 116.205) (width 0.25) (layer F.Cu) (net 17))
 (segment (start 153.416 120.65) (end 151.638 122.428) (width 0.25) (layer F.Cu) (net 17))
 (segment (start 153.416 119.507998) (end 153.416 120.65) (width 0.25) (layer F.Cu) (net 17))
 (segment (start 137.668 106.045) (end 141.605 106.045) (width 0.25) (layer F.Cu) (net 3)))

